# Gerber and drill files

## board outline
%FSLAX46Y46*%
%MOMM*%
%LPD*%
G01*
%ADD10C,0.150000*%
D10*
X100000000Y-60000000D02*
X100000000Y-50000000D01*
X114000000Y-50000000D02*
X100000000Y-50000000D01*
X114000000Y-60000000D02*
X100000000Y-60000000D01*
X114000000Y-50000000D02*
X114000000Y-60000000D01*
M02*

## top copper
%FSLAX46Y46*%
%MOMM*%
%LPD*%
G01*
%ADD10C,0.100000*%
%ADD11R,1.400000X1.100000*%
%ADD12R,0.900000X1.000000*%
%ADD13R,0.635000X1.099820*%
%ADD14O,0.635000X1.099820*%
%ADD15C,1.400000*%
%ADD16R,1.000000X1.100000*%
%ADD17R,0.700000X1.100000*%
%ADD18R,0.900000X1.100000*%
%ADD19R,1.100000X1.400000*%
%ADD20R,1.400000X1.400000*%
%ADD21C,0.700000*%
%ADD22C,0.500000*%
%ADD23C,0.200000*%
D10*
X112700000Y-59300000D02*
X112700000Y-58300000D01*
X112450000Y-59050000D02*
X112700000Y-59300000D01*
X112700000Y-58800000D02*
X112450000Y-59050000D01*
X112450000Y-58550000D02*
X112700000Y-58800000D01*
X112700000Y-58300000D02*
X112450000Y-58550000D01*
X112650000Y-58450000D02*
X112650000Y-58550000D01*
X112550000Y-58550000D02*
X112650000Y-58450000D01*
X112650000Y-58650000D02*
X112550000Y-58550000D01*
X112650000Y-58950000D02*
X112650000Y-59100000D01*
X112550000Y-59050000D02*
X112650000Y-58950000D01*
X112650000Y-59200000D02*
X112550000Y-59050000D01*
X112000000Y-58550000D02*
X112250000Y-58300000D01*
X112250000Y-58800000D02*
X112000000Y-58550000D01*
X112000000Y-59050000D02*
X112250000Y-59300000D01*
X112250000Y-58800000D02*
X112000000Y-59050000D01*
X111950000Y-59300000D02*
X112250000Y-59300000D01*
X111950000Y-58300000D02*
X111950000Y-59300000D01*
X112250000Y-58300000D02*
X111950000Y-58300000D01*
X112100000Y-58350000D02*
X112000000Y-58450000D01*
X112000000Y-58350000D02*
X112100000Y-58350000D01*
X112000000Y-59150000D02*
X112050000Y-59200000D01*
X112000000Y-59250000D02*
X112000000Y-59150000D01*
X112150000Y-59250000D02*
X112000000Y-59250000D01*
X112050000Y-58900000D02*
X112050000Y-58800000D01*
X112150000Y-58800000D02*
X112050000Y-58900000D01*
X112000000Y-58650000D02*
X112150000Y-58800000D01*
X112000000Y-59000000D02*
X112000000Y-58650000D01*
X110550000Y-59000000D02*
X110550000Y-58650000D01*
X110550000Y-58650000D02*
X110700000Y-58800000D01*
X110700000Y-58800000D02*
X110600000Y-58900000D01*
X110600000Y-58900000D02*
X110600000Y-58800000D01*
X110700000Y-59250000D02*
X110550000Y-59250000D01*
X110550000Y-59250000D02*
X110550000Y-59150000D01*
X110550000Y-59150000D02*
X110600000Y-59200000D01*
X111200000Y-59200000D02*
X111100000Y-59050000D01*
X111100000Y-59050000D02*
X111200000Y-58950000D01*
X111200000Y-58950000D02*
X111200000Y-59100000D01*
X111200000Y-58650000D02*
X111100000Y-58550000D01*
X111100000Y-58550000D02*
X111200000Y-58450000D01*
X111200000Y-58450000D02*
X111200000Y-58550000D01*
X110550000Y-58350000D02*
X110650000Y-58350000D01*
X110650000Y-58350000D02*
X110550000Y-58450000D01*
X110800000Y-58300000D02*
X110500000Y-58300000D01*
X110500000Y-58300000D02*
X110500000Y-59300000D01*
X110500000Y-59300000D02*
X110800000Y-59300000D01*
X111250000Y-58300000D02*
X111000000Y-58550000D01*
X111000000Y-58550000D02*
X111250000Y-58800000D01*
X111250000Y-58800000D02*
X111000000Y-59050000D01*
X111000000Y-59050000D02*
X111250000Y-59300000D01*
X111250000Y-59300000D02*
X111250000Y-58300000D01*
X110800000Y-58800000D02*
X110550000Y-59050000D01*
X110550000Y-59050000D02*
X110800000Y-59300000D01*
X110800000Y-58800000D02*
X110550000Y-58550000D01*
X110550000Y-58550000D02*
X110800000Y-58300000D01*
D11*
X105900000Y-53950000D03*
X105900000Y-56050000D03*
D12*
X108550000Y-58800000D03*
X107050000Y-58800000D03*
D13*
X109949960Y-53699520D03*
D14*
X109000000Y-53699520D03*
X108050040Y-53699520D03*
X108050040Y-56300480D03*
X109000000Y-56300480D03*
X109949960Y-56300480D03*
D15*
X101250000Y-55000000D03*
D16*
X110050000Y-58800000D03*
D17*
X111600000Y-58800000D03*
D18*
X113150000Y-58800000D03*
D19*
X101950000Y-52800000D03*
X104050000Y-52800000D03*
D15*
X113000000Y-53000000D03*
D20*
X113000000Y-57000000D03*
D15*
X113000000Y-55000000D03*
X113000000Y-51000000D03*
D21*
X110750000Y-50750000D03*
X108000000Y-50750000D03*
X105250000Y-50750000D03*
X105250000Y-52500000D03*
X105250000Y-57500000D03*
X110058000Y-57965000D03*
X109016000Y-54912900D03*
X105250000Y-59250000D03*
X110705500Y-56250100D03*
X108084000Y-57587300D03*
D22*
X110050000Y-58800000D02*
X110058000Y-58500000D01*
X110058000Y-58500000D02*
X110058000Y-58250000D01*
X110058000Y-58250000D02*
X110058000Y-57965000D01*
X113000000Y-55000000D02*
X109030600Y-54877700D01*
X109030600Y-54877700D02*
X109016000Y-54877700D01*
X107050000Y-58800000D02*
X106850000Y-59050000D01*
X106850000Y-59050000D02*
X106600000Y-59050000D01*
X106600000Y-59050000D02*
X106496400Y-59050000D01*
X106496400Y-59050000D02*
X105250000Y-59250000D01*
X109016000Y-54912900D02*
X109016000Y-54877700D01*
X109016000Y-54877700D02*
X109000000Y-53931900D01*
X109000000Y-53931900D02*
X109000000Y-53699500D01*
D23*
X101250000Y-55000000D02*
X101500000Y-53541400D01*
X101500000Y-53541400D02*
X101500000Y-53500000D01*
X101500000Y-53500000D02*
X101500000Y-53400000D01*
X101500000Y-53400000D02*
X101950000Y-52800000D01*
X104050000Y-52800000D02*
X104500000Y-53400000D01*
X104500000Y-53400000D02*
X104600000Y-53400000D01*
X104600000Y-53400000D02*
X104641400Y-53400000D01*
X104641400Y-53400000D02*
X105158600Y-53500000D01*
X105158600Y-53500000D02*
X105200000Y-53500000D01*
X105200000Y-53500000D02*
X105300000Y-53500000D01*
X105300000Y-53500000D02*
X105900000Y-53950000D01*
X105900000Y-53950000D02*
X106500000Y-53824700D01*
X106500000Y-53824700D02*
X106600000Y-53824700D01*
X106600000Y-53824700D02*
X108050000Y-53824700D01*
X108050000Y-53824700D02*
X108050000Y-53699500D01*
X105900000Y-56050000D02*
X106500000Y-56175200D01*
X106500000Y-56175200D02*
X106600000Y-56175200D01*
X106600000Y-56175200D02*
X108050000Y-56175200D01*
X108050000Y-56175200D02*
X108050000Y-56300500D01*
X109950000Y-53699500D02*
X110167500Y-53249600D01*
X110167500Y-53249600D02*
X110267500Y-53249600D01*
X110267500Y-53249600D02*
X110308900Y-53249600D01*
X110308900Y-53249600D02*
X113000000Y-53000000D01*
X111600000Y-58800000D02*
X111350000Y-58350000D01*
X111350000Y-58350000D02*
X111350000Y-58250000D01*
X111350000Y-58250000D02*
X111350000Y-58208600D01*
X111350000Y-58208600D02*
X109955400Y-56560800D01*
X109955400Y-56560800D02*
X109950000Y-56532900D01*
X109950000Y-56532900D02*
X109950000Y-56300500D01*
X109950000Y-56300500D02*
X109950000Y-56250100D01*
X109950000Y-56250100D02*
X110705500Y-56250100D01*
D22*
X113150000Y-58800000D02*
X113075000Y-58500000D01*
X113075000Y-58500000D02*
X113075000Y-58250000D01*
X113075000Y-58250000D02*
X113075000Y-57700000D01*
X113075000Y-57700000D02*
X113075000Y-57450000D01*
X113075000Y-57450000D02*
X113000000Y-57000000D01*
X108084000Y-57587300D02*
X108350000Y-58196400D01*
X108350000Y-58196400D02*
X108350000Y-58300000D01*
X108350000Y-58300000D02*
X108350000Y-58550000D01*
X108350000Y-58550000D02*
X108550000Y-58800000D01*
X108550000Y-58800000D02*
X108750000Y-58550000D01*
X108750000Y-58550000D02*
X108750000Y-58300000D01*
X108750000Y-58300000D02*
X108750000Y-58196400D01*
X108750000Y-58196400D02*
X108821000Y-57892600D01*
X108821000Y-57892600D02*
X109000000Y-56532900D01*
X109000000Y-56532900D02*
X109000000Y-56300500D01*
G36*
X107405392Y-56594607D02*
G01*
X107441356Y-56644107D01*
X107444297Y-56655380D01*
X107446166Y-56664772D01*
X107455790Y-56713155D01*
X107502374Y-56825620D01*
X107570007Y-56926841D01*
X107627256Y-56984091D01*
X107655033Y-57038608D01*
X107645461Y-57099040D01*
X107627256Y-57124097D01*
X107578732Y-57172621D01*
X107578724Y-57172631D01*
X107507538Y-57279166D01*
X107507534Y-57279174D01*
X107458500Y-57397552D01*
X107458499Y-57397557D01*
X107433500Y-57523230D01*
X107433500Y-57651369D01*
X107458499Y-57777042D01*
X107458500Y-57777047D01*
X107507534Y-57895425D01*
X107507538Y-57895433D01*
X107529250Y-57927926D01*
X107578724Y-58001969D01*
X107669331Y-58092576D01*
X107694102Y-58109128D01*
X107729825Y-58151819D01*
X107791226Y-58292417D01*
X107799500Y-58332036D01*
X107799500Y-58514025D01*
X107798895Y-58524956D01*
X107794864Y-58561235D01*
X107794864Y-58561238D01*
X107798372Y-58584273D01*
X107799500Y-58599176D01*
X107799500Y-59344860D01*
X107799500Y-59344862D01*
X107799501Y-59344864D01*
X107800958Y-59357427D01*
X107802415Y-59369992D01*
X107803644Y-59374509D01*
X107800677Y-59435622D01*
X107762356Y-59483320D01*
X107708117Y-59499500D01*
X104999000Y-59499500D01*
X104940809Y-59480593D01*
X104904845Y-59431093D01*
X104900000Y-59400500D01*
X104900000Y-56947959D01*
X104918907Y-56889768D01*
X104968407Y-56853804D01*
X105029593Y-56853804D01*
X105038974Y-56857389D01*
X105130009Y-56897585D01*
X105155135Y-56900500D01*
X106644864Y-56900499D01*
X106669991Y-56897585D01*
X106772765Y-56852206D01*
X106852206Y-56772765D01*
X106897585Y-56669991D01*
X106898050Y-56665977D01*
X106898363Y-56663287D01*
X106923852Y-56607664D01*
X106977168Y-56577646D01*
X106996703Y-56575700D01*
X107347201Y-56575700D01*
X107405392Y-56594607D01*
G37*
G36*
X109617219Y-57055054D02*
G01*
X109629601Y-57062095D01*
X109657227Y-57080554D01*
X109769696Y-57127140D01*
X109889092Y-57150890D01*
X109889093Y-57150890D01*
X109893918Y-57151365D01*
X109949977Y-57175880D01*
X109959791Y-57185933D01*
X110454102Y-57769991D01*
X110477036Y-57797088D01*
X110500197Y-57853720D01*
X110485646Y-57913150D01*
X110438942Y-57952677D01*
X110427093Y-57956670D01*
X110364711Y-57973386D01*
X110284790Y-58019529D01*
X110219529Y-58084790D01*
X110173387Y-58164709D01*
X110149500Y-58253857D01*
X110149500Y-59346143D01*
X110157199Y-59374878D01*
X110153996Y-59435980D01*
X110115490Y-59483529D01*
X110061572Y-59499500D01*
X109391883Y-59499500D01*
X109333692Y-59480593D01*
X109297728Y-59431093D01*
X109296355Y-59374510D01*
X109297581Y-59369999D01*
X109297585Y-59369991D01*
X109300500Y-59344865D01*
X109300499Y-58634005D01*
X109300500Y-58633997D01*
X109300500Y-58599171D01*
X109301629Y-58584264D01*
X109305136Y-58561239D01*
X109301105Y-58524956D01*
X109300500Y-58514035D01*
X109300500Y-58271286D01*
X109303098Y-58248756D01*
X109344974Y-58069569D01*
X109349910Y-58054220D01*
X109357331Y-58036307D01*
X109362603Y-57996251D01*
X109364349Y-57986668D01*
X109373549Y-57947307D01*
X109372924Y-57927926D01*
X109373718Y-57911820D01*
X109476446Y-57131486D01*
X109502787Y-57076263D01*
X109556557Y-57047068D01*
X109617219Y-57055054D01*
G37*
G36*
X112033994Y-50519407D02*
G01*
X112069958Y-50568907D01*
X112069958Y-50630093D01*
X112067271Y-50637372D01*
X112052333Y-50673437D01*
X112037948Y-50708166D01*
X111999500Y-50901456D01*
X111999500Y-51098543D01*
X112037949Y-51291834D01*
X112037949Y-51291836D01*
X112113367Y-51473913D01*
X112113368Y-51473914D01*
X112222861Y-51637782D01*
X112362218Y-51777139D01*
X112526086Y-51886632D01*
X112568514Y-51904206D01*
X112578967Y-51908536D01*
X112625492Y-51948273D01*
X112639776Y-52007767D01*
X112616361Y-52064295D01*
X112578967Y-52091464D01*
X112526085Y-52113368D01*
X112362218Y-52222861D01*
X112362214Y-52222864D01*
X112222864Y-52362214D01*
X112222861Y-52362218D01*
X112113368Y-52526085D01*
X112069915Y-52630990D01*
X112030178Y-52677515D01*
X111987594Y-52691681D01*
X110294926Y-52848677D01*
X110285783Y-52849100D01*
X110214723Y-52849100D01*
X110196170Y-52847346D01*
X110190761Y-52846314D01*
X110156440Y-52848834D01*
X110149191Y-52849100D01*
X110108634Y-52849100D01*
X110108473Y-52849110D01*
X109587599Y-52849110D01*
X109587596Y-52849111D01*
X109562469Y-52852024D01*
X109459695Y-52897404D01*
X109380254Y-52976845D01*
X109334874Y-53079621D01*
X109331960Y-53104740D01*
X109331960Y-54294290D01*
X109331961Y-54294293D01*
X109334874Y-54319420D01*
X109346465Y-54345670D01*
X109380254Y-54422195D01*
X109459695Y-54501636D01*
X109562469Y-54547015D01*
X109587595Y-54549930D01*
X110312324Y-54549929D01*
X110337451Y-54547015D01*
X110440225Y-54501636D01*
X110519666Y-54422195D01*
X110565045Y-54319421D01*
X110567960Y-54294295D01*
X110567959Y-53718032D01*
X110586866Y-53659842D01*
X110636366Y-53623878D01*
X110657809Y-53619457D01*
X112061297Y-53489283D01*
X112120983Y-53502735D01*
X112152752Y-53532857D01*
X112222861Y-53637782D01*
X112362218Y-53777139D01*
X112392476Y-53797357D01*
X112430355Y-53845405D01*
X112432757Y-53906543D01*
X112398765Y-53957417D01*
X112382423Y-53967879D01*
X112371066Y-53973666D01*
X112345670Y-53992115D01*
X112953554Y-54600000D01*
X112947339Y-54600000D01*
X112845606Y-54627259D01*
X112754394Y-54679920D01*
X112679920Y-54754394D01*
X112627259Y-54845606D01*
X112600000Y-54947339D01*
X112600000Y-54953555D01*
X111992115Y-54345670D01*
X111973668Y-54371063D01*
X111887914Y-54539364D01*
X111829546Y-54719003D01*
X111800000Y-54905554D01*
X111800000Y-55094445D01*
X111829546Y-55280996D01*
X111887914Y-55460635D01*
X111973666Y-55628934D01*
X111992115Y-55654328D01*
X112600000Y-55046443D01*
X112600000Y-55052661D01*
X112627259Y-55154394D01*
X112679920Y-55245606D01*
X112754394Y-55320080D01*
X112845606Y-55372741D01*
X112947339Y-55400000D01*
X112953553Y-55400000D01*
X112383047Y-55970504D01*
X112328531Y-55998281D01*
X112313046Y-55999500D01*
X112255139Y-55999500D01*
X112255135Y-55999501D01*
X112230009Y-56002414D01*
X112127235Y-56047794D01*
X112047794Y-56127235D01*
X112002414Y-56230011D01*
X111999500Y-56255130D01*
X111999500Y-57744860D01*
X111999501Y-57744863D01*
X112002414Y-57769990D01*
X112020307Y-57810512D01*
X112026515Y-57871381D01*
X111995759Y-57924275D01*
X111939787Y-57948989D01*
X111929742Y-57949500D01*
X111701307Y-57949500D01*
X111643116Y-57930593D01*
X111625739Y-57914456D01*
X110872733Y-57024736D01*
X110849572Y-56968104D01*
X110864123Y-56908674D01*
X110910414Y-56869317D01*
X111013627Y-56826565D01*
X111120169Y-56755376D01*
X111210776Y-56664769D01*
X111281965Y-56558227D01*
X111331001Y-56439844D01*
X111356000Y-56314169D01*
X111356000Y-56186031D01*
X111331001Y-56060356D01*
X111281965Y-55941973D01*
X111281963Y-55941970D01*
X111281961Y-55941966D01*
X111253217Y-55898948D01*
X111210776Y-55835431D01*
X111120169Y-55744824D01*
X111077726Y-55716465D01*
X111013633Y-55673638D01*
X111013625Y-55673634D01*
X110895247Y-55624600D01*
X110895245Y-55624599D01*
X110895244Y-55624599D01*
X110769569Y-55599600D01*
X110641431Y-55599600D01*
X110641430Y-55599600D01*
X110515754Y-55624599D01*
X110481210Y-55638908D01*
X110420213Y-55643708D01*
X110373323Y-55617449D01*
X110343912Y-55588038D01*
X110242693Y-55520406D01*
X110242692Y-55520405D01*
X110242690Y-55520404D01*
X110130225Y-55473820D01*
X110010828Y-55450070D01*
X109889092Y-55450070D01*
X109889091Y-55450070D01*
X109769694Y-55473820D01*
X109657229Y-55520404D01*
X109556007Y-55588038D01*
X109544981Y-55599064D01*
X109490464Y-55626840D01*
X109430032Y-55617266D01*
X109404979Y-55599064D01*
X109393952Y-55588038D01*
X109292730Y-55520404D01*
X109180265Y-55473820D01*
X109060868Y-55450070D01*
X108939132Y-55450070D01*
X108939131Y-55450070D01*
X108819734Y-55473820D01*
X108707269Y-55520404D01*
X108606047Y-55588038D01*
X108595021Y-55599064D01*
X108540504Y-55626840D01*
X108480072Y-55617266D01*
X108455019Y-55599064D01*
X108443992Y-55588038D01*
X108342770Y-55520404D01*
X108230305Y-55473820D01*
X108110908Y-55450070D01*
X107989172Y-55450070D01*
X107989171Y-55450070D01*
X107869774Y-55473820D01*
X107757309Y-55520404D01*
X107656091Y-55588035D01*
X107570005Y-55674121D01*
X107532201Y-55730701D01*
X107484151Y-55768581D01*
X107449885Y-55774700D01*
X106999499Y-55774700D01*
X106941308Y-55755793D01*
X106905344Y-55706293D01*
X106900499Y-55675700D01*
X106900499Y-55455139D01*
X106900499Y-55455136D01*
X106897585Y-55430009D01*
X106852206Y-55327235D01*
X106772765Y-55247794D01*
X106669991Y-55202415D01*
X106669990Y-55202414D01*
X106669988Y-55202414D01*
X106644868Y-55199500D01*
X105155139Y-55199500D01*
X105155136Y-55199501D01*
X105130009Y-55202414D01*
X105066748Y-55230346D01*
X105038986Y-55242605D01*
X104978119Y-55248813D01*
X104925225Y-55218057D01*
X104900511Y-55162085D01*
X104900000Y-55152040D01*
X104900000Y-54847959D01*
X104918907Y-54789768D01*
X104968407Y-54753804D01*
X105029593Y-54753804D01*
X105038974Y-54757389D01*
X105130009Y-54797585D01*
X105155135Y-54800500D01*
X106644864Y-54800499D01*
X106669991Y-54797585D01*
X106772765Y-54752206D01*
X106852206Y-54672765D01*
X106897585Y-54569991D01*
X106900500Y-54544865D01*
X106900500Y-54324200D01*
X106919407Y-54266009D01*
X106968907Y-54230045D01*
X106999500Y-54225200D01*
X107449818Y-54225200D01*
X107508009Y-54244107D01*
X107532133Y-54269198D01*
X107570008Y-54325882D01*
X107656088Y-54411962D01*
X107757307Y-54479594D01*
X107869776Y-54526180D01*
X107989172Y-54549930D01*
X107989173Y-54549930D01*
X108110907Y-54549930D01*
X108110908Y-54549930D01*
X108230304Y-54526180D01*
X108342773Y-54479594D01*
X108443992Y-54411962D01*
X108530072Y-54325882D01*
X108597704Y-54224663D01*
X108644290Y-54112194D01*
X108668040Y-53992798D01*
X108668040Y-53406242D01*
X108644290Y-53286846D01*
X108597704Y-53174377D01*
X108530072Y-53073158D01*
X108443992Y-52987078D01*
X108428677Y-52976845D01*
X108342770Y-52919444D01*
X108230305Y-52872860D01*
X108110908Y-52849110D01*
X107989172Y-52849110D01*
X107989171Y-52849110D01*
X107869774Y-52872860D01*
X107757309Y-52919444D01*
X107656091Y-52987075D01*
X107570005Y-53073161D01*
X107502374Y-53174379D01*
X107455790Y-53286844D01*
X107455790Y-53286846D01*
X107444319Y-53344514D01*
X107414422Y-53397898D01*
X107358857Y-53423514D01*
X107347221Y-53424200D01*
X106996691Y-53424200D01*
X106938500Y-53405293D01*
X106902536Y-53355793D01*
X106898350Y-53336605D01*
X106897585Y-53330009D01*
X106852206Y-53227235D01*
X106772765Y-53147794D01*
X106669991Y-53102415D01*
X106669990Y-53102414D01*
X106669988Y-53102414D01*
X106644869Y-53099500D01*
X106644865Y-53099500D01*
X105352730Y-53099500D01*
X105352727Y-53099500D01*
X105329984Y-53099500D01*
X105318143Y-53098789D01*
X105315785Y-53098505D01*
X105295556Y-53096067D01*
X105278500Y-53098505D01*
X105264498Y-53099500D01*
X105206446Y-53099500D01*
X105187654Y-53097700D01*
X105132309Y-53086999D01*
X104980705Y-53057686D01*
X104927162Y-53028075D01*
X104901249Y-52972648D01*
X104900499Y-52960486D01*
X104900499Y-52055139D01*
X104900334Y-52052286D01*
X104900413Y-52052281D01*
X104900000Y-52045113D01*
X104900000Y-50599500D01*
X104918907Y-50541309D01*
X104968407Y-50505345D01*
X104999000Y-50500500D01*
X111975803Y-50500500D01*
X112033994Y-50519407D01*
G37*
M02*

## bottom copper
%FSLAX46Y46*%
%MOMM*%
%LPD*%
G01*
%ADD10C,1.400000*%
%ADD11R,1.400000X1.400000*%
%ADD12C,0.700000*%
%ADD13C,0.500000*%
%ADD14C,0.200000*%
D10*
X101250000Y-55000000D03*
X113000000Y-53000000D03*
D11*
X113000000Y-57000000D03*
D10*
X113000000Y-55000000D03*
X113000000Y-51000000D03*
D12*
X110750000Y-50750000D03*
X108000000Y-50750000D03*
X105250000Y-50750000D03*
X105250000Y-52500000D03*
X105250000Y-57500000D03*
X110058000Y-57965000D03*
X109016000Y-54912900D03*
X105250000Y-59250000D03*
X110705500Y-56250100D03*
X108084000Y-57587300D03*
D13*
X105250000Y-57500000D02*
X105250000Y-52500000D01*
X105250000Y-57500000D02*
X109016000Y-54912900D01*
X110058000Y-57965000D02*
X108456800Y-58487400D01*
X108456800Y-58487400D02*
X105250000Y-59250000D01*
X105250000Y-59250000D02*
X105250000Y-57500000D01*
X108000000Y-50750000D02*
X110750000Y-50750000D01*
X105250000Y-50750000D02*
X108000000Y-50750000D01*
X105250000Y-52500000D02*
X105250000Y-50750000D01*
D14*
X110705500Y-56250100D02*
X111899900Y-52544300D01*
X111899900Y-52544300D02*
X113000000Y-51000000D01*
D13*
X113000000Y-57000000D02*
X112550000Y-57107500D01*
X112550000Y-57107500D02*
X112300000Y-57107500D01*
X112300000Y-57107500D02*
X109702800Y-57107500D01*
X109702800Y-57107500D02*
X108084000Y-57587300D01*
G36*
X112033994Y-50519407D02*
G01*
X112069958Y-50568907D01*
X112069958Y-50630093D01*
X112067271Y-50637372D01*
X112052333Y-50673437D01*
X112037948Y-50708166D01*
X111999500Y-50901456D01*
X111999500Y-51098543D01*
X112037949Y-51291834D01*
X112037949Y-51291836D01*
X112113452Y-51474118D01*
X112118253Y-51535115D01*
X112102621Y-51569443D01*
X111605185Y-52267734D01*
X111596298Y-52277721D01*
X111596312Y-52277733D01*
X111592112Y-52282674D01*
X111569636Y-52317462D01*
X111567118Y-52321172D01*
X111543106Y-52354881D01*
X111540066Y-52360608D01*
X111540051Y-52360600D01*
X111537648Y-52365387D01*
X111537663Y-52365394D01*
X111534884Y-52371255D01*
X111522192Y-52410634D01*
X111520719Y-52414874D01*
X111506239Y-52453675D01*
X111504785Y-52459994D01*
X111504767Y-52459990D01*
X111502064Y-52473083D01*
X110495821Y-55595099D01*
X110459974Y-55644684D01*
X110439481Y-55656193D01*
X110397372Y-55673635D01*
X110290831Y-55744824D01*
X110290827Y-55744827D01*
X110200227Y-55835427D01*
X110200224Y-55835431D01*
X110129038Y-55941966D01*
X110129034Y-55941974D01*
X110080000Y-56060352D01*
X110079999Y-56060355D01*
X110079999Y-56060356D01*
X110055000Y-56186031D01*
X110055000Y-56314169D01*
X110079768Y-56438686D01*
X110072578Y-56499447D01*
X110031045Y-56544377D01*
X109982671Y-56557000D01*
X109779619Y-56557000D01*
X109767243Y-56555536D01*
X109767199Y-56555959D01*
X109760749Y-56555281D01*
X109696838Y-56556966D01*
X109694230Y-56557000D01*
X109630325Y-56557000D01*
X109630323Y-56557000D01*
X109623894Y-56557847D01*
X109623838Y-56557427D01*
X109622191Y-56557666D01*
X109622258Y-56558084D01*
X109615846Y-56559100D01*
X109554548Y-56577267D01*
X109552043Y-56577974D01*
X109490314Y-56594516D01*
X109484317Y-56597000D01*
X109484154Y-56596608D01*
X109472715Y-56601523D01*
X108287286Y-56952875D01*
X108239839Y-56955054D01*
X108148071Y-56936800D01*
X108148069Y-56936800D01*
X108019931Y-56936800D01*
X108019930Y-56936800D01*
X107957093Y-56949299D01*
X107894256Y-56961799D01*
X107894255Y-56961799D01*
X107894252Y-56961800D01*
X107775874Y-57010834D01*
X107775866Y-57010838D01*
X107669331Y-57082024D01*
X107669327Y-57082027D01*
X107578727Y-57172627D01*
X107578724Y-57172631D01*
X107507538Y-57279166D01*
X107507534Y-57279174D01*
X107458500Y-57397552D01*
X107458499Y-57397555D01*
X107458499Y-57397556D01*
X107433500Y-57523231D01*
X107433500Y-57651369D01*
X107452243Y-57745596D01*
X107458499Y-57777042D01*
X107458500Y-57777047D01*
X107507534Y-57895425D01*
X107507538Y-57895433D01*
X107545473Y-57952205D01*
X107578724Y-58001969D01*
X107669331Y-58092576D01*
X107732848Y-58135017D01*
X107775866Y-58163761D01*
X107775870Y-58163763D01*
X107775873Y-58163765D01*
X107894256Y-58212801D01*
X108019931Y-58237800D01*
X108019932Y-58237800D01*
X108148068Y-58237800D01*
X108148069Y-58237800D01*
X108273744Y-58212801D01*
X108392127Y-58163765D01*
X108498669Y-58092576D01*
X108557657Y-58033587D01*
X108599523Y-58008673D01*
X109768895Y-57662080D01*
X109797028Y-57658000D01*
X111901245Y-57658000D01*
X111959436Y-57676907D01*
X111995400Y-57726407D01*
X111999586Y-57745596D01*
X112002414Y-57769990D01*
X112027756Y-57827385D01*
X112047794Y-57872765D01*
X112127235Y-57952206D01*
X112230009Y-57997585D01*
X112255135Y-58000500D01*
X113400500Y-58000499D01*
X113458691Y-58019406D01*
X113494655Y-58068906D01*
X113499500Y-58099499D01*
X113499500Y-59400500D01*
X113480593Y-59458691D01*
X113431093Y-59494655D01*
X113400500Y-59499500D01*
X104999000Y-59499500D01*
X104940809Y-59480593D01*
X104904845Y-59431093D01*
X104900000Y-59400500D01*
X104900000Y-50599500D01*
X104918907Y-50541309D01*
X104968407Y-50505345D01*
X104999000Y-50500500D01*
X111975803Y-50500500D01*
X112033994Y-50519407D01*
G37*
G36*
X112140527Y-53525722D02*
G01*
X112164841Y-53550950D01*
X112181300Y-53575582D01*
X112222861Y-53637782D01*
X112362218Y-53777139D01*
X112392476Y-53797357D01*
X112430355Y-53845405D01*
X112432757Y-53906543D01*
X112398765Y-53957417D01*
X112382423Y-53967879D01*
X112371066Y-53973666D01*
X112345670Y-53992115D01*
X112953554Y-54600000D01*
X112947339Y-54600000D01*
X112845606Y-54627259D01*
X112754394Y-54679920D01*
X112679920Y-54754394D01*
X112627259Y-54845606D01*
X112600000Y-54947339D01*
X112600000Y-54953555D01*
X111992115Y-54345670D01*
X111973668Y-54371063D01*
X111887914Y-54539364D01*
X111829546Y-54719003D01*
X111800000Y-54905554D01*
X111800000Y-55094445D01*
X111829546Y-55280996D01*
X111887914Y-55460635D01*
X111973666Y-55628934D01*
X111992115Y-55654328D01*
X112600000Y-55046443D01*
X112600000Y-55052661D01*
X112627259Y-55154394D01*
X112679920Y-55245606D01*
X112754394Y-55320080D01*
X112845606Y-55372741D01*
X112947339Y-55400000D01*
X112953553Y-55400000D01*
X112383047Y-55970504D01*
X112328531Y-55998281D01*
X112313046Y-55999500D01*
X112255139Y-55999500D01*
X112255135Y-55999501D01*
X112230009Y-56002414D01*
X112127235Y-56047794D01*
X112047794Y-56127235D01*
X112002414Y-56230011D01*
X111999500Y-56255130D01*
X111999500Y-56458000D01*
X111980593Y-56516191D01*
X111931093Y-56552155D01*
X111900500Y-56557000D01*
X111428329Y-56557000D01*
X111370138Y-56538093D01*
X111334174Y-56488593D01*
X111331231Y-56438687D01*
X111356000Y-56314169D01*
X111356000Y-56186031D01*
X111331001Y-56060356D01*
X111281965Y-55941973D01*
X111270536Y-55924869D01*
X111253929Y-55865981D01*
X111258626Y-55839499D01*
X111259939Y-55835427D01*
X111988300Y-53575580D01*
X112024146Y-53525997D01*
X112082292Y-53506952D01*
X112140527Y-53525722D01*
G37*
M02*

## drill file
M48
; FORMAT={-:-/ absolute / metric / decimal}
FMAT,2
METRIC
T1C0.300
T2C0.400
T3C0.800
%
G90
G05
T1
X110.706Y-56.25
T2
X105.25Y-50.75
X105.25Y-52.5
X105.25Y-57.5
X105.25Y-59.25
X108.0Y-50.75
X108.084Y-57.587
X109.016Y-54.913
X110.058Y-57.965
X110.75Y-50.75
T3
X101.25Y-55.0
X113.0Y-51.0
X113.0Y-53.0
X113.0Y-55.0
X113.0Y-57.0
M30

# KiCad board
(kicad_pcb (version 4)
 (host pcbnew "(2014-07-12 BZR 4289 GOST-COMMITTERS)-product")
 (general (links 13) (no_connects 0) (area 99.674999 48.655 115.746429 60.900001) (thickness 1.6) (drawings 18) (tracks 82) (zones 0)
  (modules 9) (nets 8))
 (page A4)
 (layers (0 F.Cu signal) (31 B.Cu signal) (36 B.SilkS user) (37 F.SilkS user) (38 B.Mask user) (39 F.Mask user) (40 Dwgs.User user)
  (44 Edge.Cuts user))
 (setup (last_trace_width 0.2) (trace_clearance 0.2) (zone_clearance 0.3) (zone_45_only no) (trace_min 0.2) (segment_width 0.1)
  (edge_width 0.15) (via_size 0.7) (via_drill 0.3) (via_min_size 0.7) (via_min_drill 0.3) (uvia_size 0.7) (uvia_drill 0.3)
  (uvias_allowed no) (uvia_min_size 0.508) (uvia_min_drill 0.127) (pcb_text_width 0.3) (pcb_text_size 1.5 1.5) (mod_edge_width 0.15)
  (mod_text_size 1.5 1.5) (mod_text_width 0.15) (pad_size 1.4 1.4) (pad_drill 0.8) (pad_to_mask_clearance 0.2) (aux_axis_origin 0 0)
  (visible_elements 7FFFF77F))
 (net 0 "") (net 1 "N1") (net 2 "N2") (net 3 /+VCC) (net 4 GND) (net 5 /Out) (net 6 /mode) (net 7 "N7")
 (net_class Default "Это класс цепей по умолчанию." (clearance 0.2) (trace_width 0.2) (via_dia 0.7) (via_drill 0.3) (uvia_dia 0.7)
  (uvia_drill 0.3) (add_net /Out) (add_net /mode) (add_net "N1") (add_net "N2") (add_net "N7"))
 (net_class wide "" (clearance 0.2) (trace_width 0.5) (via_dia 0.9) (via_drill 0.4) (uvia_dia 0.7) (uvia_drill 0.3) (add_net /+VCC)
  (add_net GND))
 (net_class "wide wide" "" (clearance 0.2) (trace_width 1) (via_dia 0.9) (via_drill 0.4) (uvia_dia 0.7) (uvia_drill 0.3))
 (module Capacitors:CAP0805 (layer F.Cu) (at 105.9 55 270)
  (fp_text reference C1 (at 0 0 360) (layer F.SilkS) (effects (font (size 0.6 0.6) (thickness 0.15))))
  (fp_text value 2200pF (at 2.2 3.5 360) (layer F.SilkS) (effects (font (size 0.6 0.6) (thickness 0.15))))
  (pad 1 smd rect (at -1.05 0 270) (size 1.1 1.4) (layers F.Cu F.Mask) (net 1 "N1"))
  (pad 2 smd rect (at 1.05 0 270) (size 1.1 1.4) (layers F.Cu F.Mask) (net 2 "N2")))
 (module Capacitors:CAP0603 (layer F.Cu) (at 107.8 58.8 180)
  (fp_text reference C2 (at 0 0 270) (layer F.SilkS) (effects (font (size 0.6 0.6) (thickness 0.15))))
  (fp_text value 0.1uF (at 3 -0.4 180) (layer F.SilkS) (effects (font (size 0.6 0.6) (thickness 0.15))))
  (pad 1 smd rect (at -0.75 0 180) (size 0.9 1) (layers F.Cu F.Mask) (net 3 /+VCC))
  (pad 2 smd rect (at 0.75 0 180) (size 0.9 1) (layers F.Cu F.Mask) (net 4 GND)))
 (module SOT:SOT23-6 (layer F.Cu) (at 109 55 180)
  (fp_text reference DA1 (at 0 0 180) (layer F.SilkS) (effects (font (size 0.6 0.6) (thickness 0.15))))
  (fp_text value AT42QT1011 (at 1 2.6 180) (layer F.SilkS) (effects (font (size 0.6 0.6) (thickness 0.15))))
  (pad 1 smd rect (at -0.94996 1.30048 180) (size 0.635 1.09982) (layers F.Cu F.Mask) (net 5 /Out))
  (pad 2 smd oval (at 0 1.30048 180) (size 0.635 1.09982) (layers F.Cu F.Mask) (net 4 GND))
  (pad 3 smd oval (at 0.94996 1.30048 180) (size 0.635 1.09982) (layers F.Cu F.Mask) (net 1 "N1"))
  (pad 4 smd oval (at 0.94996 -1.30048 180) (size 0.635 1.09982) (layers F.Cu F.Mask) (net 2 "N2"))
  (pad 5 smd oval (at 0 -1.30048 180) (size 0.635 1.09982) (layers F.Cu F.Mask) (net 3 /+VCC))
  (pad 6 smd oval (at -0.94996 -1.30048 180) (size 0.635 1.09982) (layers F.Cu F.Mask) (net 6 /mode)))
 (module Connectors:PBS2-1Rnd (layer F.Cu) (at 101.25 55)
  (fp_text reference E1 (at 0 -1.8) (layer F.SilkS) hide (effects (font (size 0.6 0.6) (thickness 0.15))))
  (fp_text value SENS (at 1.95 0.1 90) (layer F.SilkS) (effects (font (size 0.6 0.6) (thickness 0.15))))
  (pad 1 thru_hole circle (at 0 0) (size 1.4 1.4) (drill 0.8) (layers *.Cu *.Mask F.SilkS) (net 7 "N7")))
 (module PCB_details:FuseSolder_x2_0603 (layer F.Cu) (at 111.6 58.8)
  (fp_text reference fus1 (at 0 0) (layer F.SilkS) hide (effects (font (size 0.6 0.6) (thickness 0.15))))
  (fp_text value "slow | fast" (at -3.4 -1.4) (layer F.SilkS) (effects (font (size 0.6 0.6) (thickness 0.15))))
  (fp_line (start 1.1 0.5) (end 1.1 -0.5) (layer F.Cu) (width 0.1))
  (fp_line (start 0.85 0.25) (end 1.1 0.5) (layer F.Cu) (width 0.1))
  (fp_line (start 1.1 0) (end 0.85 0.25) (layer F.Cu) (width 0.1))
  (fp_line (start 0.85 -0.25) (end 1.1 0) (layer F.Cu) (width 0.1))
  (fp_line (start 1.1 -0.5) (end 0.85 -0.25) (layer F.Cu) (width 0.1))
  (fp_line (start 1.05 -0.35) (end 1.05 -0.25) (layer F.Cu) (width 0.1))
  (fp_line (start 0.95 -0.25) (end 1.05 -0.35) (layer F.Cu) (width 0.1))
  (fp_line (start 1.05 -0.15) (end 0.95 -0.25) (layer F.Cu) (width 0.1))
  (fp_line (start 1.05 0.15) (end 1.05 0.3) (layer F.Cu) (width 0.1))
  (fp_line (start 0.95 0.25) (end 1.05 0.15) (layer F.Cu) (width 0.1))
  (fp_line (start 1.05 0.4) (end 0.95 0.25) (layer F.Cu) (width 0.1))
  (fp_line (start 0.4 -0.25) (end 0.65 -0.5) (layer F.Cu) (width 0.1))
  (fp_line (start 0.65 0) (end 0.4 -0.25) (layer F.Cu) (width 0.1))
  (fp_line (start 0.4 0.25) (end 0.65 0.5) (layer F.Cu) (width 0.1))
  (fp_line (start 0.65 0) (end 0.4 0.25) (layer F.Cu) (width 0.1))
  (fp_line (start 0.35 0.5) (end 0.65 0.5) (layer F.Cu) (width 0.1))
  (fp_line (start 0.35 -0.5) (end 0.35 0.5) (layer F.Cu) (width 0.1))
  (fp_line (start 0.65 -0.5) (end 0.35 -0.5) (layer F.Cu) (width 0.1))
  (fp_line (start 0.5 -0.45) (end 0.4 -0.35) (layer F.Cu) (width 0.1))
  (fp_line (start 0.4 -0.45) (end 0.5 -0.45) (layer F.Cu) (width 0.1))
  (fp_line (start 0.4 0.35) (end 0.45 0.4) (layer F.Cu) (width 0.1))
  (fp_line (start 0.4 0.45) (end 0.4 0.35) (layer F.Cu) (width 0.1))
  (fp_line (start 0.55 0.45) (end 0.4 0.45) (layer F.Cu) (width 0.1))
  (fp_line (start 0.45 0.1) (end 0.45 0) (layer F.Cu) (width 0.1))
  (fp_line (start 0.55 0) (end 0.45 0.1) (layer F.Cu) (width 0.1))
  (fp_line (start 0.4 -0.15) (end 0.55 0) (layer F.Cu) (width 0.1))
  (fp_line (start 0.4 0.2) (end 0.4 -0.15) (layer F.Cu) (width 0.1))
  (fp_line (start -1.05 0.2) (end -1.05 -0.15) (layer F.Cu) (width 0.1))
  (fp_line (start -1.05 -0.15) (end -0.9 0) (layer F.Cu) (width 0.1))
  (fp_line (start -0.9 0) (end -1 0.1) (layer F.Cu) (width 0.1)) (fp_line (start -1 0.1) (end -1 0) (layer F.Cu) (width 0.1))
  (fp_line (start -0.9 0.45) (end -1.05 0.45) (layer F.Cu) (width 0.1))
  (fp_line (start -1.05 0.45) (end -1.05 0.35) (layer F.Cu) (width 0.1))
  (fp_line (start -1.05 0.35) (end -1 0.4) (layer F.Cu) (width 0.1))
  (fp_line (start -0.4 0.4) (end -0.5 0.25) (layer F.Cu) (width 0.1))
  (fp_line (start -0.5 0.25) (end -0.4 0.15) (layer F.Cu) (width 0.1))
  (fp_line (start -0.4 0.15) (end -0.4 0.3) (layer F.Cu) (width 0.1))
  (fp_line (start -0.4 -0.15) (end -0.5 -0.25) (layer F.Cu) (width 0.1))
  (fp_line (start -0.5 -0.25) (end -0.4 -0.35) (layer F.Cu) (width 0.1))
  (fp_line (start -0.4 -0.35) (end -0.4 -0.25) (layer F.Cu) (width 0.1))
  (fp_line (start -1.05 -0.45) (end -0.95 -0.45) (layer F.Cu) (width 0.1))
  (fp_line (start -0.95 -0.45) (end -1.05 -0.35) (layer F.Cu) (width 0.1))
  (fp_line (start -0.8 -0.5) (end -1.1 -0.5) (layer F.Cu) (width 0.1))
  (fp_line (start -1.1 -0.5) (end -1.1 0.5) (layer F.Cu) (width 0.1))
  (fp_line (start -1.1 0.5) (end -0.8 0.5) (layer F.Cu) (width 0.1))
  (fp_line (start -0.35 -0.5) (end -0.6 -0.25) (layer F.Cu) (width 0.1))
  (fp_line (start -0.6 -0.25) (end -0.35 0) (layer F.Cu) (width 0.1))
  (fp_line (start -0.35 0) (end -0.6 0.25) (layer F.Cu) (width 0.1))
  (fp_line (start -0.6 0.25) (end -0.35 0.5) (layer F.Cu) (width 0.1))
  (fp_line (start -0.35 0.5) (end -0.35 -0.5) (layer F.Cu) (width 0.1))
  (fp_line (start -0.8 0) (end -1.05 0.25) (layer F.Cu) (width 0.1))
  (fp_line (start -1.05 0.25) (end -0.8 0.5) (layer F.Cu) (width 0.1))
  (fp_line (start -0.8 0) (end -1.05 -0.25) (layer F.Cu) (width 0.1))
  (fp_line (start -1.05 -0.25) (end -0.8 -0.5) (layer F.Cu) (width 0.1))
  (pad 2 smd rect (at -1.55 0) (size 1 1.1) (layers F.Cu F.Mask) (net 4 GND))
  (pad 1 smd rect (at 0 0) (size 0.7 1.1) (layers F.Cu F.Mask) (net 6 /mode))
  (pad 3 smd rect (at 1.55 0) (size 0.9 1.1) (layers F.Cu F.Mask) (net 3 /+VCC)))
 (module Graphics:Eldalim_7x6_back (layer B.Cu) (at 107 55.4)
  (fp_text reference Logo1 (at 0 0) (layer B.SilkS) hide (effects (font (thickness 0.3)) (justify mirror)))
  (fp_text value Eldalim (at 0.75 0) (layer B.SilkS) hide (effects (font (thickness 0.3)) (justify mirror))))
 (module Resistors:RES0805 (layer F.Cu) (at 103 52.8)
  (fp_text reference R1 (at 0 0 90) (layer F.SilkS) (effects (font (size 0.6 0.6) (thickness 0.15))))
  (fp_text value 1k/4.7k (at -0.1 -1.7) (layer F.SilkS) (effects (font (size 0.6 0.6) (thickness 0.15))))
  (pad 1 smd rect (at -1.05 0) (size 1.1 1.4) (layers F.Cu F.Mask) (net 7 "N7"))
  (pad 2 smd rect (at 1.05 0) (size 1.1 1.4) (layers F.Cu F.Mask) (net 1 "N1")))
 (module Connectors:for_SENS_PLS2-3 (layer F.Cu) (at 113 57 90)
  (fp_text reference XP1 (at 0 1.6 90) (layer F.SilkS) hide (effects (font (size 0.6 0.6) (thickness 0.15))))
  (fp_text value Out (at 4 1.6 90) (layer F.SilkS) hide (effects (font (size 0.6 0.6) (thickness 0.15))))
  (pad 3 thru_hole circle (at 4 0 90) (size 1.4 1.4) (drill 0.8) (layers *.Cu *.Mask F.SilkS) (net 5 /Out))
  (pad 1 thru_hole rect (at 0 0 90) (size 1.4 1.4) (drill 0.8) (layers *.Cu *.Mask F.SilkS) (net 3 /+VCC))
  (pad 2 thru_hole circle (at 2 0 90) (size 1.4 1.4) (drill 0.8) (layers *.Cu *.Mask F.SilkS) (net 4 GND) (zone_connect 1)))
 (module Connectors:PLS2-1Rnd (layer F.Cu) (at 113 51)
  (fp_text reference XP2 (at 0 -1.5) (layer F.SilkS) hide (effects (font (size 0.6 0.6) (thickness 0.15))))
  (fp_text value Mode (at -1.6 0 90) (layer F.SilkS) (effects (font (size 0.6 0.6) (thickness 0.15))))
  (pad 1 thru_hole circle (at 0 0) (size 1.4 1.4) (drill 0.8) (layers *.Cu *.Mask F.SilkS) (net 6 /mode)))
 (gr_line (start 100 60) (end 100 50) (angle 90) (layer Edge.Cuts) (width 0.15))
 (gr_line (start 114 50) (end 100 50) (angle 90) (layer Edge.Cuts) (width 0.15))
 (gr_line (start 114 60) (end 100 60) (angle 90) (layer Edge.Cuts) (width 0.15))
 (gr_line (start 114 50) (end 114 60) (angle 90) (layer Edge.Cuts) (width 0.15))
 (segment (start 110.05 58.8) (end 110.058 58.5) (width 0.5) (layer F.Cu) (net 4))
 (segment (start 110.058 58.5) (end 110.058 58.25) (width 0.5) (layer F.Cu) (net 4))
 (segment (start 110.058 58.25) (end 110.058 57.965) (width 0.5) (layer F.Cu) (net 4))
 (segment (start 113 55) (end 109.0306 54.8777) (width 0.5) (layer F.Cu) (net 4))
 (segment (start 109.0306 54.8777) (end 109.016 54.8777) (width 0.5) (layer F.Cu) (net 4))
 (segment (start 107.05 58.8) (end 106.85 59.05) (width 0.5) (layer F.Cu) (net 4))
 (segment (start 106.85 59.05) (end 106.6 59.05) (width 0.5) (layer F.Cu) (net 4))
 (segment (start 106.6 59.05) (end 106.4964 59.05) (width 0.5) (layer F.Cu) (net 4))
 (segment (start 106.4964 59.05) (end 105.25 59.25) (width 0.5) (layer F.Cu) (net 4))
 (segment (start 109.016 54.9129) (end 109.016 54.8777) (width 0.5) (layer F.Cu) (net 4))
 (segment (start 109.016 54.8777) (end 109 53.9319) (width 0.5) (layer F.Cu) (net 4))
 (segment (start 109 53.9319) (end 109 53.6995) (width 0.5) (layer F.Cu) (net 4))
 (segment (start 105.25 57.5) (end 105.25 52.5) (width 0.5) (layer B.Cu) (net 4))
 (segment (start 105.25 57.5) (end 109.016 54.9129) (width 0.5) (layer B.Cu) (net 4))
 (segment (start 110.058 57.965) (end 108.4568 58.4874) (width 0.5) (layer B.Cu) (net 4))
 (segment (start 108.4568 58.4874) (end 105.25 59.25) (width 0.5) (layer B.Cu) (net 4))
 (segment (start 105.25 59.25) (end 105.25 57.5) (width 0.5) (layer B.Cu) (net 4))
 (segment (start 108 50.75) (end 110.75 50.75) (width 0.5) (layer B.Cu) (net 4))
 (segment (start 105.25 50.75) (end 108 50.75) (width 0.5) (layer B.Cu) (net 4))
 (segment (start 105.25 52.5) (end 105.25 50.75) (width 0.5) (layer B.Cu) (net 4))
 (via (at 110.75 50.75) (size 0.7) (layers F.Cu B.Cu) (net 4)) (via (at 108 50.75) (size 0.7) (layers F.Cu B.Cu) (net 4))
 (via (at 105.25 50.75) (size 0.7) (layers F.Cu B.Cu) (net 4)) (via (at 105.25 52.5) (size 0.7) (layers F.Cu B.Cu) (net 4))
 (via (at 105.25 57.5) (size 0.7) (layers F.Cu B.Cu) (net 4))
 (via (at 110.058 57.965) (size 0.7) (layers F.Cu B.Cu) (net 4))
 (via (at 109.016 54.9129) (size 0.7) (layers F.Cu B.Cu) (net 4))
 (via (at 105.25 59.25) (size 0.7) (layers F.Cu B.Cu) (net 4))
 (segment (start 101.25 55) (end 101.5 53.5414) (width 0.2) (layer F.Cu) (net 7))
 (segment (start 101.5 53.5414) (end 101.5 53.5) (width 0.2) (layer F.Cu) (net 7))
 (segment (start 101.5 53.5) (end 101.5 53.4) (width 0.2) (layer F.Cu) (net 7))
 (segment (start 101.5 53.4) (end 101.95 52.8) (width 0.2) (layer F.Cu) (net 7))
 (segment (start 104.05 52.8) (end 104.5 53.4) (width 0.2) (layer F.Cu) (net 1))
 (segment (start 104.5 53.4) (end 104.6 53.4) (width 0.2) (layer F.Cu) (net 1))
 (segment (start 104.6 53.4) (end 104.6414 53.4) (width 0.2) (layer F.Cu) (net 1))
 (segment (start 104.6414 53.4) (end 105.1586 53.5) (width 0.2) (layer F.Cu) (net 1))
 (segment (start 105.1586 53.5) (end 105.2 53.5) (width 0.2) (layer F.Cu) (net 1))
 (segment (start 105.2 53.5) (end 105.3 53.5) (width 0.2) (layer F.Cu) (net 1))
 (segment (start 105.3 53.5) (end 105.9 53.95) (width 0.2) (layer F.Cu) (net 1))
 (segment (start 105.9 53.95) (end 106.5 53.8247) (width 0.2) (layer F.Cu) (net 1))
 (segment (start 106.5 53.8247) (end 106.6 53.8247) (width 0.2) (layer F.Cu) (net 1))
 (segment (start 106.6 53.8247) (end 108.05 53.8247) (width 0.2) (layer F.Cu) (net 1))
 (segment (start 108.05 53.8247) (end 108.05 53.6995) (width 0.2) (layer F.Cu) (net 1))
 (segment (start 105.9 56.05) (end 106.5 56.1752) (width 0.2) (layer F.Cu) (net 2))
 (segment (start 106.5 56.1752) (end 106.6 56.1752) (width 0.2) (layer F.Cu) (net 2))
 (segment (start 106.6 56.1752) (end 108.05 56.1752) (width 0.2) (layer F.Cu) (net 2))
 (segment (start 108.05 56.1752) (end 108.05 56.3005) (width 0.2) (layer F.Cu) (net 2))
 (segment (start 109.95 53.6995) (end 110.1675 53.2496) (width 0.2) (layer F.Cu) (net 5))
 (segment (start 110.1675 53.2496) (end 110.2675 53.2496) (width 0.2) (layer F.Cu) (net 5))
 (segment (start 110.2675 53.2496) (end 110.3089 53.2496) (width 0.2) (layer F.Cu) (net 5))
 (segment (start 110.3089 53.2496) (end 113 53) (width 0.2) (layer F.Cu) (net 5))
 (segment (start 111.6 58.8) (end 111.35 58.35) (width 0.2) (layer F.Cu) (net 6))
 (segment (start 111.35 58.35) (end 111.35 58.25) (width 0.2) (layer F.Cu) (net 6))
 (segment (start 111.35 58.25) (end 111.35 58.2086) (width 0.2) (layer F.Cu) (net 6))
 (segment (start 111.35 58.2086) (end 109.9554 56.5608) (width 0.2) (layer F.Cu) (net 6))
 (segment (start 109.9554 56.5608) (end 109.95 56.5329) (width 0.2) (layer F.Cu) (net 6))
 (segment (start 109.95 56.5329) (end 109.95 56.3005) (width 0.2) (layer F.Cu) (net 6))
 (segment (start 109.95 56.3005) (end 109.95 56.2501) (width 0.2) (layer F.Cu) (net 6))
 (segment (start 109.95 56.2501) (end 110.7055 56.2501) (width 0.2) (layer F.Cu) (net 6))
 (segment (start 110.7055 56.2501) (end 111.8999 52.5443) (width 0.2) (layer B.Cu) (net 6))
 (segment (start 111.8999 52.5443) (end 113 51) (width 0.2) (layer B.Cu) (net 6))
 (via (at 110.7055 56.2501) (size 0.7) (layers F.Cu B.Cu) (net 6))
 (segment (start 113.15 58.8) (end 113.075 58.5) (width 0.5) (layer F.Cu) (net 3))
 (segment (start 113.075 58.5) (end 113.075 58.25) (width 0.5) (layer F.Cu) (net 3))
 (segment (start 113.075 58.25) (end 113.075 57.7) (width 0.5) (layer F.Cu) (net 3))
 (segment (start 113.075 57.7) (end 113.075 57.45) (width 0.5) (layer F.Cu) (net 3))
 (segment (start 113.075 57.45) (end 113 57) (width 0.5) (layer F.Cu) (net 3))
 (segment (start 108.084 57.5873) (end 108.35 58.1964) (width 0.5) (layer F.Cu) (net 3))
 (segment (start 108.35 58.1964) (end 108.35 58.3) (width 0.5) (layer F.Cu) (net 3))
 (segment (start 108.35 58.3) (end 108.35 58.55) (width 0.5) (layer F.Cu) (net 3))
 (segment (start 108.35 58.55) (end 108.55 58.8) (width 0.5) (layer F.Cu) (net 3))
 (segment (start 108.55 58.8) (end 108.75 58.55) (width 0.5) (layer F.Cu) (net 3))
 (segment (start 108.75 58.55) (end 108.75 58.3) (width 0.5) (layer F.Cu) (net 3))
 (segment (start 108.75 58.3) (end 108.75 58.1964) (width 0.5) (layer F.Cu) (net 3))
 (segment (start 108.75 58.1964) (end 108.821 57.8926) (width 0.5) (layer F.Cu) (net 3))
 (segment (start 108.821 57.8926) (end 109 56.5329) (width 0.5) (layer F.Cu) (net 3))
 (segment (start 109 56.5329) (end 109 56.3005) (width 0.5) (layer F.Cu) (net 3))
 (segment (start 113 57) (end 112.55 57.1075) (width 0.5) (layer B.Cu) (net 3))
 (segment (start 112.55 57.1075) (end 112.3 57.1075) (width 0.5) (layer B.Cu) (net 3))
 (segment (start 112.3 57.1075) (end 109.7028 57.1075) (width 0.5) (layer B.Cu) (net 3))
 (segment (start 109.7028 57.1075) (end 108.084 57.5873) (width 0.5) (layer B.Cu) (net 3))
 (via (at 108.084 57.5873) (size 0.7) (layers F.Cu B.Cu) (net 3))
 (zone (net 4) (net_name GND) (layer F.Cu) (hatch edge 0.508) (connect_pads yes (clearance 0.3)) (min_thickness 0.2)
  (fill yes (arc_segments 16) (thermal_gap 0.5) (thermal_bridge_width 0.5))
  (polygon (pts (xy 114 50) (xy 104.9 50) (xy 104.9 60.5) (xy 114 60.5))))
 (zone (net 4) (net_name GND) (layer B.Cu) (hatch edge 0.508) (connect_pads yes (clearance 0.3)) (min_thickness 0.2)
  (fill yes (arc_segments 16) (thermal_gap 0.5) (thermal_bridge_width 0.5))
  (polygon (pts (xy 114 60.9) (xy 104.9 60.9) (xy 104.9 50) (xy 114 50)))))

